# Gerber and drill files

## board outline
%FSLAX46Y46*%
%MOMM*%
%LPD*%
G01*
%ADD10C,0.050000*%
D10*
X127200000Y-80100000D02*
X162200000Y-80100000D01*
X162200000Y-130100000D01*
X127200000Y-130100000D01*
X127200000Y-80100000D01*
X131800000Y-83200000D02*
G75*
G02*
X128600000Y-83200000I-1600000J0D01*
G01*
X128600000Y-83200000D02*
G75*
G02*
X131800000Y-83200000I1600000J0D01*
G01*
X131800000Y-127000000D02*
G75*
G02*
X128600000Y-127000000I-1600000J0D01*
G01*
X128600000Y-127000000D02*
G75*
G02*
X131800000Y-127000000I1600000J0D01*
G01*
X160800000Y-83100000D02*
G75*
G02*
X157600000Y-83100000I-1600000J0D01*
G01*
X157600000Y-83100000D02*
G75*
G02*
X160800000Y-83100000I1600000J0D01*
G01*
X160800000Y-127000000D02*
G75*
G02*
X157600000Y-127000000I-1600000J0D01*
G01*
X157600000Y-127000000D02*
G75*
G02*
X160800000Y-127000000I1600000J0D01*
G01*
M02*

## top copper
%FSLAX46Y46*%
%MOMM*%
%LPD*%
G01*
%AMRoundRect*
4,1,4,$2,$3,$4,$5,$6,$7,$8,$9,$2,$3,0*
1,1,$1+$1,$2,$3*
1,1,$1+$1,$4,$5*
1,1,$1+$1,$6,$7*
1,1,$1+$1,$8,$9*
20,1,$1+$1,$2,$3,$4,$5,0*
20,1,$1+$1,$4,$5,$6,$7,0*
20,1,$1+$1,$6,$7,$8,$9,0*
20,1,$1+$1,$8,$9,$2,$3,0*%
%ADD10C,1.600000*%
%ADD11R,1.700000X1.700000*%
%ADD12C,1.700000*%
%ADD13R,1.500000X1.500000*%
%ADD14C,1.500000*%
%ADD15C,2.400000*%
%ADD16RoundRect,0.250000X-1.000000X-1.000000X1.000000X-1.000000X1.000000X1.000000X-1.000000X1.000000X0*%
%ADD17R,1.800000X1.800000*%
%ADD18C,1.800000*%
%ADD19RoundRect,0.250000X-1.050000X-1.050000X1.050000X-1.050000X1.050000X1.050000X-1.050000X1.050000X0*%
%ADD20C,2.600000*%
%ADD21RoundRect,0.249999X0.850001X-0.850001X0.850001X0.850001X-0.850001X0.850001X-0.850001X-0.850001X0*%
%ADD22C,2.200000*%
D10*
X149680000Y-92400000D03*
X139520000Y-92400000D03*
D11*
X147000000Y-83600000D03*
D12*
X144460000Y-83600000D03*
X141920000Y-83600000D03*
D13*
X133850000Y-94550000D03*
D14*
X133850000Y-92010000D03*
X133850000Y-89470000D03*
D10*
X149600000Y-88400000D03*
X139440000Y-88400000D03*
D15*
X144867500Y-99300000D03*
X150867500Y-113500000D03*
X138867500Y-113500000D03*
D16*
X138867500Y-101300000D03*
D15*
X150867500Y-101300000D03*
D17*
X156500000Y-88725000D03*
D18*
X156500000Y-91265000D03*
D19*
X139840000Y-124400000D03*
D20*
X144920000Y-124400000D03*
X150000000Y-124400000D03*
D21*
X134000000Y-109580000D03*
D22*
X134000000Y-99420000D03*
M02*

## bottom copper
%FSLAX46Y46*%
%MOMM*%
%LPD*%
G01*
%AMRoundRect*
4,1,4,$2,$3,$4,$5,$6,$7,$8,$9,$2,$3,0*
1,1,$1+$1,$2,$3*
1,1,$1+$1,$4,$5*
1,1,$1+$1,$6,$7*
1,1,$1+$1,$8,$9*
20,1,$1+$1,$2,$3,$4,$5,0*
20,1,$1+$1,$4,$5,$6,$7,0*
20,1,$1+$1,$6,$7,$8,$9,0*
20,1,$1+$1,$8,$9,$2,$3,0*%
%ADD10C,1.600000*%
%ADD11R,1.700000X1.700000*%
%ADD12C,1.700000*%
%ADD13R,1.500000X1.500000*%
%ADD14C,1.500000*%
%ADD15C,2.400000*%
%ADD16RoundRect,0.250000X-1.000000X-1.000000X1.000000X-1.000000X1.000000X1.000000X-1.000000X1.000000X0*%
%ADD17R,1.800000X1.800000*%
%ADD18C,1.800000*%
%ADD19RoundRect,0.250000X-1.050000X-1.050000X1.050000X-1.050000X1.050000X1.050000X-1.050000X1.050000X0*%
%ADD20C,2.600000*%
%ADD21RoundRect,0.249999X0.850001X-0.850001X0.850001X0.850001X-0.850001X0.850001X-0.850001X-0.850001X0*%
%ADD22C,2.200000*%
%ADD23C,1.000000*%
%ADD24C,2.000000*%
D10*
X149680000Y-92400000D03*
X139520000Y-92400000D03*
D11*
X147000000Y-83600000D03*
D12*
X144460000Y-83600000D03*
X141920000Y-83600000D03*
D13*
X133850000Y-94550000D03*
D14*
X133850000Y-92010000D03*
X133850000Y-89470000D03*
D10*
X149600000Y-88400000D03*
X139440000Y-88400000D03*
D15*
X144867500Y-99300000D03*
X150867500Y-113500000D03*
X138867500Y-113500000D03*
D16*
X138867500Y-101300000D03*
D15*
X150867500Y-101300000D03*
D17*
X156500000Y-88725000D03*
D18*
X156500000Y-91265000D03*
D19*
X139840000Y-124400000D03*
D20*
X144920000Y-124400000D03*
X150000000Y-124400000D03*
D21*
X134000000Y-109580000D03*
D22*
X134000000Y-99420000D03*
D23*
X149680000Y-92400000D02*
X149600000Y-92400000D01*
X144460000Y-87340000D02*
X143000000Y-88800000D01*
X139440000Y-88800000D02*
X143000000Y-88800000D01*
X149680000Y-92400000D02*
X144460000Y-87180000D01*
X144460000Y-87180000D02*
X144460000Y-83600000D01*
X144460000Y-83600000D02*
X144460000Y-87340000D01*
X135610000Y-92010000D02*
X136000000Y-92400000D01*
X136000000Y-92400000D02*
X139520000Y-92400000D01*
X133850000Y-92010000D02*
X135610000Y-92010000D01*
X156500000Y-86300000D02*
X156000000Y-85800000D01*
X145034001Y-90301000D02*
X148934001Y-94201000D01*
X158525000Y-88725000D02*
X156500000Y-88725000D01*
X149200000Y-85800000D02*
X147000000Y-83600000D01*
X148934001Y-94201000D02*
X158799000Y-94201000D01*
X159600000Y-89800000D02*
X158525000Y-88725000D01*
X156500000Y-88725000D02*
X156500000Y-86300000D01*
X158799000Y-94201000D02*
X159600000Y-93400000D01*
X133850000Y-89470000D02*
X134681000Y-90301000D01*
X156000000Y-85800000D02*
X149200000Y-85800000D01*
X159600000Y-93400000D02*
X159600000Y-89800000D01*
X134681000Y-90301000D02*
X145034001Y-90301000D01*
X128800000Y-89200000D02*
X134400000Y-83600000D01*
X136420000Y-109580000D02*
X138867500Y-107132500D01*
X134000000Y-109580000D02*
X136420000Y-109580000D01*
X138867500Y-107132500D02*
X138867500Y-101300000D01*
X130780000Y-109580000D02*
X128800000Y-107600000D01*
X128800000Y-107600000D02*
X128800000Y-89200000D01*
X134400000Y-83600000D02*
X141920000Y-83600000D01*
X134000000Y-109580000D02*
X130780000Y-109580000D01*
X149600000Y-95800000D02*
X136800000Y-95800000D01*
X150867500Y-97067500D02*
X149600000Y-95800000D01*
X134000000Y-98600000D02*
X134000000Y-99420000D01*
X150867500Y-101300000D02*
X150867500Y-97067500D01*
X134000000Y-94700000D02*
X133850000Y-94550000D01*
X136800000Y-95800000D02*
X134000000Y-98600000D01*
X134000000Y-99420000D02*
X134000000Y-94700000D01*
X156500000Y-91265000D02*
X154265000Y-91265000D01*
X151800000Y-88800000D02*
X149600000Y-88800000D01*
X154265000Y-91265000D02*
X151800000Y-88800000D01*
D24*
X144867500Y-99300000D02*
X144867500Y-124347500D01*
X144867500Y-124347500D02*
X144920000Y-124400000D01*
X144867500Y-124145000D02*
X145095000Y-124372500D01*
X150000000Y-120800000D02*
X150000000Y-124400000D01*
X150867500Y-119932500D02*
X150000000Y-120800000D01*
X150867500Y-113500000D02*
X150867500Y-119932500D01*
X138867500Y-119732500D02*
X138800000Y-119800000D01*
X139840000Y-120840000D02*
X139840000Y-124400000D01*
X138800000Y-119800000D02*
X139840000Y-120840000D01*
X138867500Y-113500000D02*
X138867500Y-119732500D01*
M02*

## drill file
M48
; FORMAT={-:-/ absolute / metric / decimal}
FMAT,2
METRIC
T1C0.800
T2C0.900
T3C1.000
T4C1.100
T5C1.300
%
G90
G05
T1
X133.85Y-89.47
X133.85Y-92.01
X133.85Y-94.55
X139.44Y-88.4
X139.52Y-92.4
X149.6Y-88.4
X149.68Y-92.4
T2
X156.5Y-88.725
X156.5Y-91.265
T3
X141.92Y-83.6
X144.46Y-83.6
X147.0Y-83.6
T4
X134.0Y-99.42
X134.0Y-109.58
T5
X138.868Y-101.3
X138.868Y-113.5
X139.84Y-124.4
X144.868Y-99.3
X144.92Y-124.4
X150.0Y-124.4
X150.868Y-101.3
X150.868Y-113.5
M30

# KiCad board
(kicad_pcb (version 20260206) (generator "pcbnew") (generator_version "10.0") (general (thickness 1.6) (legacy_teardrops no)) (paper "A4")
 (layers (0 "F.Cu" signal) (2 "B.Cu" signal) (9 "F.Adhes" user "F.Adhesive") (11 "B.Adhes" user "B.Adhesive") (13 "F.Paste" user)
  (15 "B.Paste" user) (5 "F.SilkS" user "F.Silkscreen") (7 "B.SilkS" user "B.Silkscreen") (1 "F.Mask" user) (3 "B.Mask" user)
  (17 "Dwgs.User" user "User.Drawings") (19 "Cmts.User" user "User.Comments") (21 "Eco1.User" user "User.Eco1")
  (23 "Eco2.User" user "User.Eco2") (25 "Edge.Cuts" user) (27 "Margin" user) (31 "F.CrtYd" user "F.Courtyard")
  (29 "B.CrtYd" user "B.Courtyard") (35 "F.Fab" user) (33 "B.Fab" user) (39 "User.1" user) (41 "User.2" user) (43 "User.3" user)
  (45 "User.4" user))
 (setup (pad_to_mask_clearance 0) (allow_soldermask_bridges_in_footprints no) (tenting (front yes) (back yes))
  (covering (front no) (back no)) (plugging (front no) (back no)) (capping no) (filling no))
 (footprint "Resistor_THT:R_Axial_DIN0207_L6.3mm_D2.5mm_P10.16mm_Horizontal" (layer "F.Cu") (at 149.68 92.4 180)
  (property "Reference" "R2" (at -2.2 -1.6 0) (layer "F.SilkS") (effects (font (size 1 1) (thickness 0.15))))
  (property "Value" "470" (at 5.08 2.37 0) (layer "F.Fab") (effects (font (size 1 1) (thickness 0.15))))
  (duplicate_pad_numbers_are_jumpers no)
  (pad "1" thru_hole circle (at 0 0 180) (size 1.6 1.6) (drill 0.8) (layers "*.Cu" "*.Mask") (remove_unused_layers no) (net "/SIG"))
  (pad "2" thru_hole circle (at 10.16 0 180) (size 1.6 1.6) (drill 0.8) (layers "*.Cu" "*.Mask") (remove_unused_layers no) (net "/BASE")))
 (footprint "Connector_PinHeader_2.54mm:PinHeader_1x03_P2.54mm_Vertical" (layer "F.Cu") (at 147 83.6 -90)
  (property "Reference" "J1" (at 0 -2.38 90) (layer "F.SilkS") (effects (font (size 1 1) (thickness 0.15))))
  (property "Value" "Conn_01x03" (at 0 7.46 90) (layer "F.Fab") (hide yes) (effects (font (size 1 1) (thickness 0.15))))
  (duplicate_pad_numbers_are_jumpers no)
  (pad "1" thru_hole rect (at 0 0 270) (size 1.7 1.7) (drill 1) (layers "*.Cu" "*.Mask") (remove_unused_layers no) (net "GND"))
  (pad "2" thru_hole circle (at 0 2.54 270) (size 1.7 1.7) (drill 1) (layers "*.Cu" "*.Mask") (remove_unused_layers no) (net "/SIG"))
  (pad "3" thru_hole circle (at 0 5.08 270) (size 1.7 1.7) (drill 1) (layers "*.Cu" "*.Mask") (remove_unused_layers no) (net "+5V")))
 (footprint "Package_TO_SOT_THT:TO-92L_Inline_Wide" (layer "F.Cu") (at 133.85 94.55 90)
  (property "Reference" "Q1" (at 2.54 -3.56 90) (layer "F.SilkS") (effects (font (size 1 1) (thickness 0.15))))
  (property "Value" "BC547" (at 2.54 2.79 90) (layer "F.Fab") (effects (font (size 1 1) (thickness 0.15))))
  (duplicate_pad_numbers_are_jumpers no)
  (pad "1" thru_hole rect (at 0 0 90) (size 1.5 1.5) (drill 0.8) (layers "*.Cu" "*.Mask") (remove_unused_layers no) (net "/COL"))
  (pad "2" thru_hole circle (at 2.54 0 90) (size 1.5 1.5) (drill 0.8) (layers "*.Cu" "*.Mask") (remove_unused_layers no) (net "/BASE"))
  (pad "3" thru_hole circle (at 5.08 0 90) (size 1.5 1.5) (drill 0.8) (layers "*.Cu" "*.Mask") (remove_unused_layers no) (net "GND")))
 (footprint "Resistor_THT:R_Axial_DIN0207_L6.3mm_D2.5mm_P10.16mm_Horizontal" (layer "F.Cu") (at 149.6 88.4 180)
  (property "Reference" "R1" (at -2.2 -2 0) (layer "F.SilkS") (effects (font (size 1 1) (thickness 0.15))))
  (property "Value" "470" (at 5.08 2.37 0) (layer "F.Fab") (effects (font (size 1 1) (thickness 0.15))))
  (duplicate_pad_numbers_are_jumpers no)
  (pad "1" thru_hole circle (at 0 0 180) (size 1.6 1.6) (drill 0.8) (layers "*.Cu" "*.Mask") (remove_unused_layers no) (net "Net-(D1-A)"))
  (pad "2" thru_hole circle (at 10.16 0 180) (size 1.6 1.6) (drill 0.8) (layers "*.Cu" "*.Mask") (remove_unused_layers no) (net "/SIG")))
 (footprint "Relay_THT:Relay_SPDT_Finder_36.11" (layer "F.Cu") (at 138.8675 101.3)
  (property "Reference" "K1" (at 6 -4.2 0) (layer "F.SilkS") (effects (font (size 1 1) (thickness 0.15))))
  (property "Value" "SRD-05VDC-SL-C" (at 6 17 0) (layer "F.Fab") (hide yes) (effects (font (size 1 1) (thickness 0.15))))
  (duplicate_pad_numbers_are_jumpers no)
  (pad "11" thru_hole circle (at 6 -2) (size 2.4 2.4) (drill 1.3) (layers "*.Cu" "*.Mask") (remove_unused_layers no) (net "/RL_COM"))
  (pad "12" thru_hole circle (at 12 12.2) (size 2.4 2.4) (drill 1.3) (layers "*.Cu" "*.Mask") (remove_unused_layers no) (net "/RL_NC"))
  (pad "14" thru_hole circle (at 0 12.2) (size 2.4 2.4) (drill 1.3) (layers "*.Cu" "*.Mask") (remove_unused_layers no) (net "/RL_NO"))
  (pad "A1" thru_hole roundrect (at 0 0) (size 2.5 2.5) (drill 1.3) (layers "*.Cu" "*.Mask") (remove_unused_layers no)
   (roundrect_rratio 0.1) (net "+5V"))
  (pad "A2" thru_hole circle (at 12 0) (size 2.4 2.4) (drill 1.3) (layers "*.Cu" "*.Mask") (remove_unused_layers no) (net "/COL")))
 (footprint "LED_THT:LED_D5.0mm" (layer "F.Cu") (at 156.5 88.725 -90)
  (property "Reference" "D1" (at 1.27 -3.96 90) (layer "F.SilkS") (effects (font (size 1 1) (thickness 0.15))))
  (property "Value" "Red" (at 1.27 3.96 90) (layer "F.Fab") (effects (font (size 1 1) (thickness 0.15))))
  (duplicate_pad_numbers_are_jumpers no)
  (pad "1" thru_hole rect (at 0 0 270) (size 1.8 1.8) (drill 0.9) (layers "*.Cu" "*.Mask") (remove_unused_layers no) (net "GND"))
  (pad "2" thru_hole circle (at 2.54 0 270) (size 1.8 1.8) (drill 0.9) (layers "*.Cu" "*.Mask") (remove_unused_layers no) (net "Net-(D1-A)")))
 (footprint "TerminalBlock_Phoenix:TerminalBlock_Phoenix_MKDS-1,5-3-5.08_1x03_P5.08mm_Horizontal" (layer "F.Cu") (at 139.84 124.4)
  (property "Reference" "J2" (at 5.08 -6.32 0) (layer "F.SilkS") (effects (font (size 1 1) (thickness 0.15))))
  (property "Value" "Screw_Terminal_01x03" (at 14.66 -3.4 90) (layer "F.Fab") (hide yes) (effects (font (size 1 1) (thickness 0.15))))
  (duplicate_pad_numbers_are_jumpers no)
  (pad "1" thru_hole roundrect (at 0 0) (size 2.6 2.6) (drill 1.3) (layers "*.Cu" "*.Mask") (remove_unused_layers no)
   (roundrect_rratio 0.096154) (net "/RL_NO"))
  (pad "2" thru_hole circle (at 5.08 0) (size 2.6 2.6) (drill 1.3) (layers "*.Cu" "*.Mask") (remove_unused_layers no) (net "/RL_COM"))
  (pad "3" thru_hole circle (at 10.16 0) (size 2.6 2.6) (drill 1.3) (layers "*.Cu" "*.Mask") (remove_unused_layers no) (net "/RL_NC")))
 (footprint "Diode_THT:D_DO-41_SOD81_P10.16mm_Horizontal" (layer "F.Cu") (at 134 109.58 90)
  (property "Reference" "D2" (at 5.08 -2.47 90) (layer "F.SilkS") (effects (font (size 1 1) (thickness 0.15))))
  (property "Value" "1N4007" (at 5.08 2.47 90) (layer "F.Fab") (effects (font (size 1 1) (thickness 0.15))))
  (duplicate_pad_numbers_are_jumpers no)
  (pad "1" thru_hole roundrect (at 0 0 90) (size 2.2 2.2) (drill 1.1) (layers "*.Cu" "*.Mask") (remove_unused_layers no)
   (roundrect_rratio 0.113636) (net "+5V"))
  (pad "2" thru_hole circle (at 10.16 0 90) (size 2.2 2.2) (drill 1.1) (layers "*.Cu" "*.Mask") (remove_unused_layers no) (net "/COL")))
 (gr_rect (start 127.2 80.1) (end 162.2 130.1) (stroke (width 0.05) (type solid)) (fill no) (layer "Edge.Cuts"))
 (gr_circle (center 130.2 83.2) (end 131.8 83.2) (stroke (width 0.05) (type default)) (fill no) (layer "Edge.Cuts"))
 (gr_circle (center 130.2 127) (end 131.8 127) (stroke (width 0.05) (type default)) (fill no) (layer "Edge.Cuts"))
 (gr_circle (center 159.2 83.1) (end 160.8 83.1) (stroke (width 0.05) (type default)) (fill no) (layer "Edge.Cuts"))
 (gr_circle (center 159.2 127) (end 160.8 127) (stroke (width 0.05) (type default)) (fill no) (layer "Edge.Cuts"))
 (segment (start 149.68 92.4) (end 149.6 92.4) (width 1) (layer "B.Cu") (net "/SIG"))
 (segment (start 144.46 87.34) (end 143 88.8) (width 1) (layer "B.Cu") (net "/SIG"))
 (segment (start 139.44 88.8) (end 143 88.8) (width 1) (layer "B.Cu") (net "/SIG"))
 (segment (start 149.68 92.4) (end 144.46 87.18) (width 1) (layer "B.Cu") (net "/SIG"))
 (segment (start 144.46 87.18) (end 144.46 83.6) (width 1) (layer "B.Cu") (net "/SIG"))
 (segment (start 144.46 83.6) (end 144.46 87.34) (width 1) (layer "B.Cu") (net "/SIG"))
 (segment (start 135.61 92.01) (end 136 92.4) (width 1) (layer "B.Cu") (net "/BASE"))
 (segment (start 136 92.4) (end 139.52 92.4) (width 1) (layer "B.Cu") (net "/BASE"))
 (segment (start 133.85 92.01) (end 135.61 92.01) (width 1) (layer "B.Cu") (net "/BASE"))
 (segment (start 156.5 86.3) (end 156 85.8) (width 1) (layer "B.Cu") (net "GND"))
 (segment (start 145.034001 90.301) (end 148.934001 94.201) (width 1) (layer "B.Cu") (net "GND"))
 (segment (start 158.525 88.725) (end 156.5 88.725) (width 1) (layer "B.Cu") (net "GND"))
 (segment (start 149.2 85.8) (end 147 83.6) (width 1) (layer "B.Cu") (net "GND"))
 (segment (start 148.934001 94.201) (end 158.799 94.201) (width 1) (layer "B.Cu") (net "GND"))
 (segment (start 159.6 89.8) (end 158.525 88.725) (width 1) (layer "B.Cu") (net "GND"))
 (segment (start 156.5 88.725) (end 156.5 86.3) (width 1) (layer "B.Cu") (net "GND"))
 (segment (start 158.799 94.201) (end 159.6 93.4) (width 1) (layer "B.Cu") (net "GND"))
 (segment (start 133.85 89.47) (end 134.681 90.301) (width 1) (layer "B.Cu") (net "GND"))
 (segment (start 156 85.8) (end 149.2 85.8) (width 1) (layer "B.Cu") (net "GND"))
 (segment (start 159.6 93.4) (end 159.6 89.8) (width 1) (layer "B.Cu") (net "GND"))
 (segment (start 134.681 90.301) (end 145.034001 90.301) (width 1) (layer "B.Cu") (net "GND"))
 (segment (start 128.8 89.2) (end 134.4 83.6) (width 1) (layer "B.Cu") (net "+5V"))
 (segment (start 136.42 109.58) (end 138.8675 107.1325) (width 1) (layer "B.Cu") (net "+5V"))
 (segment (start 134 109.58) (end 136.42 109.58) (width 1) (layer "B.Cu") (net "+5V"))
 (segment (start 138.8675 107.1325) (end 138.8675 101.3) (width 1) (layer "B.Cu") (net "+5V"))
 (segment (start 130.78 109.58) (end 128.8 107.6) (width 1) (layer "B.Cu") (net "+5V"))
 (segment (start 128.8 107.6) (end 128.8 89.2) (width 1) (layer "B.Cu") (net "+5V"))
 (segment (start 134.4 83.6) (end 141.92 83.6) (width 1) (layer "B.Cu") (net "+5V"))
 (segment (start 134 109.58) (end 130.78 109.58) (width 1) (layer "B.Cu") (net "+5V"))
 (segment (start 149.6 95.8) (end 136.8 95.8) (width 1) (layer "B.Cu") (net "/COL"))
 (segment (start 150.8675 97.0675) (end 149.6 95.8) (width 1) (layer "B.Cu") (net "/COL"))
 (segment (start 134 98.6) (end 134 99.42) (width 1) (layer "B.Cu") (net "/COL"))
 (segment (start 150.8675 101.3) (end 150.8675 97.0675) (width 1) (layer "B.Cu") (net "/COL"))
 (segment (start 134 94.7) (end 133.85 94.55) (width 1) (layer "B.Cu") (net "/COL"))
 (segment (start 136.8 95.8) (end 134 98.6) (width 1) (layer "B.Cu") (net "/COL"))
 (segment (start 134 99.42) (end 134 94.7) (width 1) (layer "B.Cu") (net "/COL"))
 (segment (start 156.5 91.265) (end 154.265 91.265) (width 1) (layer "B.Cu") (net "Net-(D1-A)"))
 (segment (start 151.8 88.8) (end 149.6 88.8) (width 1) (layer "B.Cu") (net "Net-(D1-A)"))
 (segment (start 154.265 91.265) (end 151.8 88.8) (width 1) (layer "B.Cu") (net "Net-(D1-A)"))
 (segment (start 144.8675 99.3) (end 144.8675 124.3475) (width 2) (layer "B.Cu") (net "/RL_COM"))
 (segment (start 144.8675 124.3475) (end 144.92 124.4) (width 2) (layer "B.Cu") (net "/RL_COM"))
 (segment (start 144.8675 124.145) (end 145.095 124.3725) (width 2) (layer "B.Cu") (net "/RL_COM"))
 (segment (start 150 120.8) (end 150 124.4) (width 2) (layer "B.Cu") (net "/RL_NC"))
 (segment (start 150.8675 119.9325) (end 150 120.8) (width 2) (layer "B.Cu") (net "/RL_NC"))
 (segment (start 150.8675 113.5) (end 150.8675 119.9325) (width 2) (layer "B.Cu") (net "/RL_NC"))
 (segment (start 138.8675 119.7325) (end 138.8 119.8) (width 2) (layer "B.Cu") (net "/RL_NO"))
 (segment (start 139.84 120.84) (end 139.84 124.4) (width 2) (layer "B.Cu") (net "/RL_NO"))
 (segment (start 138.8 119.8) (end 139.84 120.84) (width 2) (layer "B.Cu") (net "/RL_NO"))
 (segment (start 138.8675 113.5) (end 138.8675 119.7325) (width 2) (layer "B.Cu") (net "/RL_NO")))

